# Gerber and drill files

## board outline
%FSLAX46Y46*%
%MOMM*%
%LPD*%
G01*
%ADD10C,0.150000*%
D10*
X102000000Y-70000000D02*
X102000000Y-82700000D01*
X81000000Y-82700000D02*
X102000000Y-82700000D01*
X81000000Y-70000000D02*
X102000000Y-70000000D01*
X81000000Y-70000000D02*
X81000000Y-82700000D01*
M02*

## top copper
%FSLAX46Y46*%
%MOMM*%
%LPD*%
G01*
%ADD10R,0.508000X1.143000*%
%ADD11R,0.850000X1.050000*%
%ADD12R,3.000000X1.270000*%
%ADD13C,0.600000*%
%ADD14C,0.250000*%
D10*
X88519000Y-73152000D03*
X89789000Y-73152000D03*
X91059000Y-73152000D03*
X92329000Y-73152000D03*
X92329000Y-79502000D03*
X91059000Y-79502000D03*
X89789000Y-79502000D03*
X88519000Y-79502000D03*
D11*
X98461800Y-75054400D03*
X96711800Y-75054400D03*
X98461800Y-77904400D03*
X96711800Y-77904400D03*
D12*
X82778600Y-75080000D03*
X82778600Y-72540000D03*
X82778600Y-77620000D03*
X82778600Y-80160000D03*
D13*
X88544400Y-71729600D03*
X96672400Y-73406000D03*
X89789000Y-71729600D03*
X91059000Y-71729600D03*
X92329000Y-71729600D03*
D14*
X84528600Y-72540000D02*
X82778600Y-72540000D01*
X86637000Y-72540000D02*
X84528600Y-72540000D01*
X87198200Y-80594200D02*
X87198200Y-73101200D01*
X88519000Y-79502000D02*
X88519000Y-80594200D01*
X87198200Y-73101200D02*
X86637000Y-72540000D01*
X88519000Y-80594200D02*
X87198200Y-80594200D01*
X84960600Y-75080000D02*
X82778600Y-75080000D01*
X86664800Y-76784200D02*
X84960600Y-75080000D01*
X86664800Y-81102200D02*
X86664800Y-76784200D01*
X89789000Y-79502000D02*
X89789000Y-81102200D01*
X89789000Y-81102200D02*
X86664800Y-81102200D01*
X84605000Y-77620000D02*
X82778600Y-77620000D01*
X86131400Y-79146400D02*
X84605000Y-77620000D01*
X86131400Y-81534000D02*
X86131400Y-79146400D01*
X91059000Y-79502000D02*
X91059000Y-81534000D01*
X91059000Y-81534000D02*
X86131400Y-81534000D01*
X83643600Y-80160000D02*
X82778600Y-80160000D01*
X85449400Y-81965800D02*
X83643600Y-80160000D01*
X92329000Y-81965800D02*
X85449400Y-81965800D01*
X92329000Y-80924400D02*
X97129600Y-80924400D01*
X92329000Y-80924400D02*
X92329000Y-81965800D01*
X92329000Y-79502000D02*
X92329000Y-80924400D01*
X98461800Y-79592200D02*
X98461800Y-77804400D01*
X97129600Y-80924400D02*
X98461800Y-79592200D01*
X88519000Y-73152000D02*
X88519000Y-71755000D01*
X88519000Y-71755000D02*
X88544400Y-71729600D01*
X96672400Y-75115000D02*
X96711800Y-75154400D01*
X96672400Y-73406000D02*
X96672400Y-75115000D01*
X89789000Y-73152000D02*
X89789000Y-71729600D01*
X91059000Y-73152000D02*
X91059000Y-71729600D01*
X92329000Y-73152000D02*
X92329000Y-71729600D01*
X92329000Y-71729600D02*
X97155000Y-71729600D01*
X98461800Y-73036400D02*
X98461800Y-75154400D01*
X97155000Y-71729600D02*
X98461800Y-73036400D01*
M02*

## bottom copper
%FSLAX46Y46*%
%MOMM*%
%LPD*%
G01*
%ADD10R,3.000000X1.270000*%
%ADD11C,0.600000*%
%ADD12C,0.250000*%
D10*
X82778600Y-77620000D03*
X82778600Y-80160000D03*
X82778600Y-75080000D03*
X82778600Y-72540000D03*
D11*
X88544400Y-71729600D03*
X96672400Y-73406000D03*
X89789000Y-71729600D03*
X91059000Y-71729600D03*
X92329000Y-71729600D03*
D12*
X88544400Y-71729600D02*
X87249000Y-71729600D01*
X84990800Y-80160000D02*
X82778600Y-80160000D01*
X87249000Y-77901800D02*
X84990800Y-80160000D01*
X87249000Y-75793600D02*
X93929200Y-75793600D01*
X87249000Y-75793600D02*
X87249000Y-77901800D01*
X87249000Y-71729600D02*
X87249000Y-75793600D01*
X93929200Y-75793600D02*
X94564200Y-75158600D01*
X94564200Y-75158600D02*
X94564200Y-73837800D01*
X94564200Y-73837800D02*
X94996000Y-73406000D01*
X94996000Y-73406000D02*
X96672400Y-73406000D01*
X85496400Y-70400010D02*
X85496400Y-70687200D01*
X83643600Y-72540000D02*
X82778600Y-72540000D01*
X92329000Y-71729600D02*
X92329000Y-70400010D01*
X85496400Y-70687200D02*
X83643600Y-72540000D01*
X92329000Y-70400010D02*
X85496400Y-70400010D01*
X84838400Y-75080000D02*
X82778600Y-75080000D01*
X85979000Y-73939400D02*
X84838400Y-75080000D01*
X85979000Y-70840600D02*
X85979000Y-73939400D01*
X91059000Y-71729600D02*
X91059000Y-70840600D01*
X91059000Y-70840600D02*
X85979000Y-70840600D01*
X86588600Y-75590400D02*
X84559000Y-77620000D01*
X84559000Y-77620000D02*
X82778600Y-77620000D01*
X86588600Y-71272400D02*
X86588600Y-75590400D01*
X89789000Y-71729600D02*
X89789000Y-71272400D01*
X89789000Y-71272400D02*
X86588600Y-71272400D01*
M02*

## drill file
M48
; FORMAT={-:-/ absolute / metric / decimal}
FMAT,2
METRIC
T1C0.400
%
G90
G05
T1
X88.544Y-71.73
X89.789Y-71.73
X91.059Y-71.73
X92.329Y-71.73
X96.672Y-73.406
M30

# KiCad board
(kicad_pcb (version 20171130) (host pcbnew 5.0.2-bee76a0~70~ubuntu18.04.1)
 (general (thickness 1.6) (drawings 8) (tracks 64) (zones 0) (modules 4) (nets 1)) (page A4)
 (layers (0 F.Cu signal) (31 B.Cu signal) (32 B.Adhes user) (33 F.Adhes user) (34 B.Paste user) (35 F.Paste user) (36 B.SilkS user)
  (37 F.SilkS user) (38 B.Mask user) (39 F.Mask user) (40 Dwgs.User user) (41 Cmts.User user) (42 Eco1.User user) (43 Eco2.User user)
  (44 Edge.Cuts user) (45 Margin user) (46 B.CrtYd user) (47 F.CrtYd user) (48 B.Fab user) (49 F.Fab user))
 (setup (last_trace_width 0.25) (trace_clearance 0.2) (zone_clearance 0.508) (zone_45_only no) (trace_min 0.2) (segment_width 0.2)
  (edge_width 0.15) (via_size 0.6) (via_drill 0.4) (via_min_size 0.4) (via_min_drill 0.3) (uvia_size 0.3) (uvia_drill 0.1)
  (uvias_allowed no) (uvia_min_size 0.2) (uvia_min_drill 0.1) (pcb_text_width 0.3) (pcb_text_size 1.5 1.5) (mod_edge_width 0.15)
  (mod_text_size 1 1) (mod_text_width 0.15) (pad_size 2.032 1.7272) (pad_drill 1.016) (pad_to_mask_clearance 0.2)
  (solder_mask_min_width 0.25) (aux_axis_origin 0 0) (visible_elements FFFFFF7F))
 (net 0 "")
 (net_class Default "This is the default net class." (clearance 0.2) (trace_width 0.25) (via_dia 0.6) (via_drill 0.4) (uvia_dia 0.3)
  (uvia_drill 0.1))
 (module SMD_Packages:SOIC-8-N (layer F.Cu) (at 90.424 76.327)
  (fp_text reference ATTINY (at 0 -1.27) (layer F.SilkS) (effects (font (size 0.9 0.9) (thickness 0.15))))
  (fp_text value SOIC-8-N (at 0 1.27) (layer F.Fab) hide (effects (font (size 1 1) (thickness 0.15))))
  (pad 8 smd rect (at -1.905 -3.175) (size 0.508 1.143) (layers F.Cu F.Paste F.Mask))
  (pad 7 smd rect (at -0.635 -3.175) (size 0.508 1.143) (layers F.Cu F.Paste F.Mask))
  (pad 6 smd rect (at 0.635 -3.175) (size 0.508 1.143) (layers F.Cu F.Paste F.Mask))
  (pad 5 smd rect (at 1.905 -3.175) (size 0.508 1.143) (layers F.Cu F.Paste F.Mask))
  (pad 4 smd rect (at 1.905 3.175) (size 0.508 1.143) (layers F.Cu F.Paste F.Mask))
  (pad 3 smd rect (at 0.635 3.175) (size 0.508 1.143) (layers F.Cu F.Paste F.Mask))
  (pad 2 smd rect (at -0.635 3.175) (size 0.508 1.143) (layers F.Cu F.Paste F.Mask))
  (pad 1 smd rect (at -1.905 3.175) (size 0.508 1.143) (layers F.Cu F.Paste F.Mask)))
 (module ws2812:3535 (layer F.Cu) (at 97.5868 76.4794 90)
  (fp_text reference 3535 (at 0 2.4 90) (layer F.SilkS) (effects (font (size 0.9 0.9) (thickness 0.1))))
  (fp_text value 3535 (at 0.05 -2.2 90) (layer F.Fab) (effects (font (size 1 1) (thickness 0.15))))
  (pad IN smd rect (at 1.325 0.875 90) (size 1.05 0.85) (drill (offset 0.1 0)) (layers F.Cu F.Paste F.Mask))
  (pad VDD smd rect (at 1.325 -0.875 90) (size 1.05 0.85) (drill (offset 0.1 0)) (layers F.Cu F.Paste F.Mask))
  (pad GND smd rect (at -1.325 0.875 90) (size 1.05 0.85) (drill (offset -0.1 0)) (layers F.Cu F.Paste F.Mask))
  (pad OUT smd rect (at -1.325 -0.875 90) (size 1.05 0.85) (drill (offset -0.1 0)) (layers F.Cu F.Paste F.Mask)))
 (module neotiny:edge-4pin (layer F.Cu) (at 82.7786 80.16 90)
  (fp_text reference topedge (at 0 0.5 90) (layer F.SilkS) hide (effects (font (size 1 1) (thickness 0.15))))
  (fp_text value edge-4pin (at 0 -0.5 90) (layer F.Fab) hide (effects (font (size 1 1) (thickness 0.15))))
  (pad 3 connect rect (at 5.08 0 90) (size 1.27 3) (layers F.Cu F.Mask))
  (pad 4 connect rect (at 7.62 0 90) (size 1.27 3) (layers F.Cu F.Mask))
  (pad 2 connect rect (at 2.54 0 90) (size 1.27 3) (layers F.Cu F.Mask))
  (pad 1 connect rect (at 0 0 90) (size 1.27 3) (layers F.Cu F.Mask)))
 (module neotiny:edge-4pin (layer B.Cu) (at 82.7786 72.54 270)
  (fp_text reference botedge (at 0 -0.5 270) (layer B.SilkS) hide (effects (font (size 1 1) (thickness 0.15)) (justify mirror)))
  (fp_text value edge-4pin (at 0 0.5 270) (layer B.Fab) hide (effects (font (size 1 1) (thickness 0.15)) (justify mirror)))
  (pad 3 connect rect (at 5.08 0 270) (size 1.27 3) (layers B.Cu B.Mask))
  (pad 4 connect rect (at 7.62 0 270) (size 1.27 3) (layers B.Cu B.Mask))
  (pad 2 connect rect (at 2.54 0 270) (size 1.27 3) (layers B.Cu B.Mask))
  (pad 1 connect rect (at 0 0 270) (size 1.27 3) (layers B.Cu B.Mask)))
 (gr_line (start 102 70) (end 102 82.7) (angle 90) (layer Edge.Cuts) (width 0.15))
 (gr_line (start 81 82.7) (end 102 82.7) (angle 90) (layer Edge.Cuts) (width 0.15))
 (gr_line (start 81 70) (end 102 70) (angle 90) (layer Edge.Cuts) (width 0.15))
 (gr_line (start 81 70) (end 81 82.7) (angle 90) (layer Edge.Cuts) (width 0.15))
 (segment (start 84.5286 72.54) (end 82.7786 72.54) (width 0.25) (layer F.Cu) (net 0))
 (segment (start 86.637 72.54) (end 84.5286 72.54) (width 0.25) (layer F.Cu) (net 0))
 (segment (start 87.1982 80.5942) (end 87.1982 73.1012) (width 0.25) (layer F.Cu) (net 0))
 (segment (start 88.519 79.502) (end 88.519 80.5942) (width 0.25) (layer F.Cu) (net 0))
 (segment (start 87.1982 73.1012) (end 86.637 72.54) (width 0.25) (layer F.Cu) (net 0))
 (segment (start 88.519 80.5942) (end 87.1982 80.5942) (width 0.25) (layer F.Cu) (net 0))
 (segment (start 84.9606 75.08) (end 82.7786 75.08) (width 0.25) (layer F.Cu) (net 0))
 (segment (start 86.6648 76.7842) (end 84.9606 75.08) (width 0.25) (layer F.Cu) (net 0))
 (segment (start 86.6648 81.1022) (end 86.6648 76.7842) (width 0.25) (layer F.Cu) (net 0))
 (segment (start 89.789 79.502) (end 89.789 81.1022) (width 0.25) (layer F.Cu) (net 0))
 (segment (start 89.789 81.1022) (end 86.6648 81.1022) (width 0.25) (layer F.Cu) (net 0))
 (segment (start 84.605 77.62) (end 82.7786 77.62) (width 0.25) (layer F.Cu) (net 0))
 (segment (start 86.1314 79.1464) (end 84.605 77.62) (width 0.25) (layer F.Cu) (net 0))
 (segment (start 86.1314 81.534) (end 86.1314 79.1464) (width 0.25) (layer F.Cu) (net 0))
 (segment (start 91.059 79.502) (end 91.059 81.534) (width 0.25) (layer F.Cu) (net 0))
 (segment (start 91.059 81.534) (end 86.1314 81.534) (width 0.25) (layer F.Cu) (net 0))
 (segment (start 83.6436 80.16) (end 82.7786 80.16) (width 0.25) (layer F.Cu) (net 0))
 (segment (start 85.4494 81.9658) (end 83.6436 80.16) (width 0.25) (layer F.Cu) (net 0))
 (segment (start 92.329 81.9658) (end 85.4494 81.9658) (width 0.25) (layer F.Cu) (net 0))
 (segment (start 92.329 80.9244) (end 97.1296 80.9244) (width 0.25) (layer F.Cu) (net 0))
 (segment (start 92.329 80.9244) (end 92.329 81.9658) (width 0.25) (layer F.Cu) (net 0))
 (segment (start 92.329 79.502) (end 92.329 80.9244) (width 0.25) (layer F.Cu) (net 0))
 (segment (start 98.4618 79.5922) (end 98.4618 77.8044) (width 0.25) (layer F.Cu) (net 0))
 (segment (start 97.1296 80.9244) (end 98.4618 79.5922) (width 0.25) (layer F.Cu) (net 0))
 (via (at 88.5444 71.7296) (size 0.6) (drill 0.4) (layers F.Cu B.Cu) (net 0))
 (segment (start 88.519 73.152) (end 88.519 71.755) (width 0.25) (layer F.Cu) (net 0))
 (segment (start 88.519 71.755) (end 88.5444 71.7296) (width 0.25) (layer F.Cu) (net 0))
 (segment (start 88.5444 71.7296) (end 87.249 71.7296) (width 0.25) (layer B.Cu) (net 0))
 (segment (start 84.9908 80.16) (end 82.7786 80.16) (width 0.25) (layer B.Cu) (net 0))
 (segment (start 87.249 77.9018) (end 84.9908 80.16) (width 0.25) (layer B.Cu) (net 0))
 (segment (start 87.249 75.7936) (end 93.9292 75.7936) (width 0.25) (layer B.Cu) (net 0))
 (segment (start 87.249 75.7936) (end 87.249 77.9018) (width 0.25) (layer B.Cu) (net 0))
 (segment (start 87.249 71.7296) (end 87.249 75.7936) (width 0.25) (layer B.Cu) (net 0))
 (segment (start 93.9292 75.7936) (end 94.5642 75.1586) (width 0.25) (layer B.Cu) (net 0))
 (segment (start 94.5642 75.1586) (end 94.5642 73.8378) (width 0.25) (layer B.Cu) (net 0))
 (segment (start 94.5642 73.8378) (end 94.996 73.406) (width 0.25) (layer B.Cu) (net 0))
 (via (at 96.6724 73.406) (size 0.6) (drill 0.4) (layers F.Cu B.Cu) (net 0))
 (segment (start 94.996 73.406) (end 96.6724 73.406) (width 0.25) (layer B.Cu) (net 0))
 (segment (start 96.6724 75.115) (end 96.7118 75.1544) (width 0.25) (layer F.Cu) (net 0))
 (segment (start 96.6724 73.406) (end 96.6724 75.115) (width 0.25) (layer F.Cu) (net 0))
 (via (at 89.789 71.7296) (size 0.6) (drill 0.4) (layers F.Cu B.Cu) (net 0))
 (segment (start 89.789 73.152) (end 89.789 71.7296) (width 0.25) (layer F.Cu) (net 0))
 (via (at 91.059 71.7296) (size 0.6) (drill 0.4) (layers F.Cu B.Cu) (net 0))
 (segment (start 91.059 73.152) (end 91.059 71.7296) (width 0.25) (layer F.Cu) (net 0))
 (via (at 92.329 71.7296) (size 0.6) (drill 0.4) (layers F.Cu B.Cu) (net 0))
 (segment (start 92.329 73.152) (end 92.329 71.7296) (width 0.25) (layer F.Cu) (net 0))
 (segment (start 85.4964 70.40001) (end 85.4964 70.6872) (width 0.25) (layer B.Cu) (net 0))
 (segment (start 83.6436 72.54) (end 82.7786 72.54) (width 0.25) (layer B.Cu) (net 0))
 (segment (start 92.329 71.7296) (end 92.329 70.40001) (width 0.25) (layer B.Cu) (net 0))
 (segment (start 85.4964 70.6872) (end 83.6436 72.54) (width 0.25) (layer B.Cu) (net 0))
 (segment (start 92.329 70.40001) (end 85.4964 70.40001) (width 0.25) (layer B.Cu) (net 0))
 (segment (start 84.8384 75.08) (end 82.7786 75.08) (width 0.25) (layer B.Cu) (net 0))
 (segment (start 85.979 73.9394) (end 84.8384 75.08) (width 0.25) (layer B.Cu) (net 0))
 (segment (start 85.979 70.8406) (end 85.979 73.9394) (width 0.25) (layer B.Cu) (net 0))
 (segment (start 91.059 71.7296) (end 91.059 70.8406) (width 0.25) (layer B.Cu) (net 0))
 (segment (start 91.059 70.8406) (end 85.979 70.8406) (width 0.25) (layer B.Cu) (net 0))
 (segment (start 86.5886 75.5904) (end 84.559 77.62) (width 0.25) (layer B.Cu) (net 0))
 (segment (start 84.559 77.62) (end 82.7786 77.62) (width 0.25) (layer B.Cu) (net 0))
 (segment (start 86.5886 71.2724) (end 86.5886 75.5904) (width 0.25) (layer B.Cu) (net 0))
 (segment (start 89.789 71.7296) (end 89.789 71.2724) (width 0.25) (layer B.Cu) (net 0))
 (segment (start 89.789 71.2724) (end 86.5886 71.2724) (width 0.25) (layer B.Cu) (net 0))
 (segment (start 92.329 71.7296) (end 97.155 71.7296) (width 0.25) (layer F.Cu) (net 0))
 (segment (start 98.4618 73.0364) (end 98.4618 75.1544) (width 0.25) (layer F.Cu) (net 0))
 (segment (start 97.155 71.7296) (end 98.4618 73.0364) (width 0.25) (layer F.Cu) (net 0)))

